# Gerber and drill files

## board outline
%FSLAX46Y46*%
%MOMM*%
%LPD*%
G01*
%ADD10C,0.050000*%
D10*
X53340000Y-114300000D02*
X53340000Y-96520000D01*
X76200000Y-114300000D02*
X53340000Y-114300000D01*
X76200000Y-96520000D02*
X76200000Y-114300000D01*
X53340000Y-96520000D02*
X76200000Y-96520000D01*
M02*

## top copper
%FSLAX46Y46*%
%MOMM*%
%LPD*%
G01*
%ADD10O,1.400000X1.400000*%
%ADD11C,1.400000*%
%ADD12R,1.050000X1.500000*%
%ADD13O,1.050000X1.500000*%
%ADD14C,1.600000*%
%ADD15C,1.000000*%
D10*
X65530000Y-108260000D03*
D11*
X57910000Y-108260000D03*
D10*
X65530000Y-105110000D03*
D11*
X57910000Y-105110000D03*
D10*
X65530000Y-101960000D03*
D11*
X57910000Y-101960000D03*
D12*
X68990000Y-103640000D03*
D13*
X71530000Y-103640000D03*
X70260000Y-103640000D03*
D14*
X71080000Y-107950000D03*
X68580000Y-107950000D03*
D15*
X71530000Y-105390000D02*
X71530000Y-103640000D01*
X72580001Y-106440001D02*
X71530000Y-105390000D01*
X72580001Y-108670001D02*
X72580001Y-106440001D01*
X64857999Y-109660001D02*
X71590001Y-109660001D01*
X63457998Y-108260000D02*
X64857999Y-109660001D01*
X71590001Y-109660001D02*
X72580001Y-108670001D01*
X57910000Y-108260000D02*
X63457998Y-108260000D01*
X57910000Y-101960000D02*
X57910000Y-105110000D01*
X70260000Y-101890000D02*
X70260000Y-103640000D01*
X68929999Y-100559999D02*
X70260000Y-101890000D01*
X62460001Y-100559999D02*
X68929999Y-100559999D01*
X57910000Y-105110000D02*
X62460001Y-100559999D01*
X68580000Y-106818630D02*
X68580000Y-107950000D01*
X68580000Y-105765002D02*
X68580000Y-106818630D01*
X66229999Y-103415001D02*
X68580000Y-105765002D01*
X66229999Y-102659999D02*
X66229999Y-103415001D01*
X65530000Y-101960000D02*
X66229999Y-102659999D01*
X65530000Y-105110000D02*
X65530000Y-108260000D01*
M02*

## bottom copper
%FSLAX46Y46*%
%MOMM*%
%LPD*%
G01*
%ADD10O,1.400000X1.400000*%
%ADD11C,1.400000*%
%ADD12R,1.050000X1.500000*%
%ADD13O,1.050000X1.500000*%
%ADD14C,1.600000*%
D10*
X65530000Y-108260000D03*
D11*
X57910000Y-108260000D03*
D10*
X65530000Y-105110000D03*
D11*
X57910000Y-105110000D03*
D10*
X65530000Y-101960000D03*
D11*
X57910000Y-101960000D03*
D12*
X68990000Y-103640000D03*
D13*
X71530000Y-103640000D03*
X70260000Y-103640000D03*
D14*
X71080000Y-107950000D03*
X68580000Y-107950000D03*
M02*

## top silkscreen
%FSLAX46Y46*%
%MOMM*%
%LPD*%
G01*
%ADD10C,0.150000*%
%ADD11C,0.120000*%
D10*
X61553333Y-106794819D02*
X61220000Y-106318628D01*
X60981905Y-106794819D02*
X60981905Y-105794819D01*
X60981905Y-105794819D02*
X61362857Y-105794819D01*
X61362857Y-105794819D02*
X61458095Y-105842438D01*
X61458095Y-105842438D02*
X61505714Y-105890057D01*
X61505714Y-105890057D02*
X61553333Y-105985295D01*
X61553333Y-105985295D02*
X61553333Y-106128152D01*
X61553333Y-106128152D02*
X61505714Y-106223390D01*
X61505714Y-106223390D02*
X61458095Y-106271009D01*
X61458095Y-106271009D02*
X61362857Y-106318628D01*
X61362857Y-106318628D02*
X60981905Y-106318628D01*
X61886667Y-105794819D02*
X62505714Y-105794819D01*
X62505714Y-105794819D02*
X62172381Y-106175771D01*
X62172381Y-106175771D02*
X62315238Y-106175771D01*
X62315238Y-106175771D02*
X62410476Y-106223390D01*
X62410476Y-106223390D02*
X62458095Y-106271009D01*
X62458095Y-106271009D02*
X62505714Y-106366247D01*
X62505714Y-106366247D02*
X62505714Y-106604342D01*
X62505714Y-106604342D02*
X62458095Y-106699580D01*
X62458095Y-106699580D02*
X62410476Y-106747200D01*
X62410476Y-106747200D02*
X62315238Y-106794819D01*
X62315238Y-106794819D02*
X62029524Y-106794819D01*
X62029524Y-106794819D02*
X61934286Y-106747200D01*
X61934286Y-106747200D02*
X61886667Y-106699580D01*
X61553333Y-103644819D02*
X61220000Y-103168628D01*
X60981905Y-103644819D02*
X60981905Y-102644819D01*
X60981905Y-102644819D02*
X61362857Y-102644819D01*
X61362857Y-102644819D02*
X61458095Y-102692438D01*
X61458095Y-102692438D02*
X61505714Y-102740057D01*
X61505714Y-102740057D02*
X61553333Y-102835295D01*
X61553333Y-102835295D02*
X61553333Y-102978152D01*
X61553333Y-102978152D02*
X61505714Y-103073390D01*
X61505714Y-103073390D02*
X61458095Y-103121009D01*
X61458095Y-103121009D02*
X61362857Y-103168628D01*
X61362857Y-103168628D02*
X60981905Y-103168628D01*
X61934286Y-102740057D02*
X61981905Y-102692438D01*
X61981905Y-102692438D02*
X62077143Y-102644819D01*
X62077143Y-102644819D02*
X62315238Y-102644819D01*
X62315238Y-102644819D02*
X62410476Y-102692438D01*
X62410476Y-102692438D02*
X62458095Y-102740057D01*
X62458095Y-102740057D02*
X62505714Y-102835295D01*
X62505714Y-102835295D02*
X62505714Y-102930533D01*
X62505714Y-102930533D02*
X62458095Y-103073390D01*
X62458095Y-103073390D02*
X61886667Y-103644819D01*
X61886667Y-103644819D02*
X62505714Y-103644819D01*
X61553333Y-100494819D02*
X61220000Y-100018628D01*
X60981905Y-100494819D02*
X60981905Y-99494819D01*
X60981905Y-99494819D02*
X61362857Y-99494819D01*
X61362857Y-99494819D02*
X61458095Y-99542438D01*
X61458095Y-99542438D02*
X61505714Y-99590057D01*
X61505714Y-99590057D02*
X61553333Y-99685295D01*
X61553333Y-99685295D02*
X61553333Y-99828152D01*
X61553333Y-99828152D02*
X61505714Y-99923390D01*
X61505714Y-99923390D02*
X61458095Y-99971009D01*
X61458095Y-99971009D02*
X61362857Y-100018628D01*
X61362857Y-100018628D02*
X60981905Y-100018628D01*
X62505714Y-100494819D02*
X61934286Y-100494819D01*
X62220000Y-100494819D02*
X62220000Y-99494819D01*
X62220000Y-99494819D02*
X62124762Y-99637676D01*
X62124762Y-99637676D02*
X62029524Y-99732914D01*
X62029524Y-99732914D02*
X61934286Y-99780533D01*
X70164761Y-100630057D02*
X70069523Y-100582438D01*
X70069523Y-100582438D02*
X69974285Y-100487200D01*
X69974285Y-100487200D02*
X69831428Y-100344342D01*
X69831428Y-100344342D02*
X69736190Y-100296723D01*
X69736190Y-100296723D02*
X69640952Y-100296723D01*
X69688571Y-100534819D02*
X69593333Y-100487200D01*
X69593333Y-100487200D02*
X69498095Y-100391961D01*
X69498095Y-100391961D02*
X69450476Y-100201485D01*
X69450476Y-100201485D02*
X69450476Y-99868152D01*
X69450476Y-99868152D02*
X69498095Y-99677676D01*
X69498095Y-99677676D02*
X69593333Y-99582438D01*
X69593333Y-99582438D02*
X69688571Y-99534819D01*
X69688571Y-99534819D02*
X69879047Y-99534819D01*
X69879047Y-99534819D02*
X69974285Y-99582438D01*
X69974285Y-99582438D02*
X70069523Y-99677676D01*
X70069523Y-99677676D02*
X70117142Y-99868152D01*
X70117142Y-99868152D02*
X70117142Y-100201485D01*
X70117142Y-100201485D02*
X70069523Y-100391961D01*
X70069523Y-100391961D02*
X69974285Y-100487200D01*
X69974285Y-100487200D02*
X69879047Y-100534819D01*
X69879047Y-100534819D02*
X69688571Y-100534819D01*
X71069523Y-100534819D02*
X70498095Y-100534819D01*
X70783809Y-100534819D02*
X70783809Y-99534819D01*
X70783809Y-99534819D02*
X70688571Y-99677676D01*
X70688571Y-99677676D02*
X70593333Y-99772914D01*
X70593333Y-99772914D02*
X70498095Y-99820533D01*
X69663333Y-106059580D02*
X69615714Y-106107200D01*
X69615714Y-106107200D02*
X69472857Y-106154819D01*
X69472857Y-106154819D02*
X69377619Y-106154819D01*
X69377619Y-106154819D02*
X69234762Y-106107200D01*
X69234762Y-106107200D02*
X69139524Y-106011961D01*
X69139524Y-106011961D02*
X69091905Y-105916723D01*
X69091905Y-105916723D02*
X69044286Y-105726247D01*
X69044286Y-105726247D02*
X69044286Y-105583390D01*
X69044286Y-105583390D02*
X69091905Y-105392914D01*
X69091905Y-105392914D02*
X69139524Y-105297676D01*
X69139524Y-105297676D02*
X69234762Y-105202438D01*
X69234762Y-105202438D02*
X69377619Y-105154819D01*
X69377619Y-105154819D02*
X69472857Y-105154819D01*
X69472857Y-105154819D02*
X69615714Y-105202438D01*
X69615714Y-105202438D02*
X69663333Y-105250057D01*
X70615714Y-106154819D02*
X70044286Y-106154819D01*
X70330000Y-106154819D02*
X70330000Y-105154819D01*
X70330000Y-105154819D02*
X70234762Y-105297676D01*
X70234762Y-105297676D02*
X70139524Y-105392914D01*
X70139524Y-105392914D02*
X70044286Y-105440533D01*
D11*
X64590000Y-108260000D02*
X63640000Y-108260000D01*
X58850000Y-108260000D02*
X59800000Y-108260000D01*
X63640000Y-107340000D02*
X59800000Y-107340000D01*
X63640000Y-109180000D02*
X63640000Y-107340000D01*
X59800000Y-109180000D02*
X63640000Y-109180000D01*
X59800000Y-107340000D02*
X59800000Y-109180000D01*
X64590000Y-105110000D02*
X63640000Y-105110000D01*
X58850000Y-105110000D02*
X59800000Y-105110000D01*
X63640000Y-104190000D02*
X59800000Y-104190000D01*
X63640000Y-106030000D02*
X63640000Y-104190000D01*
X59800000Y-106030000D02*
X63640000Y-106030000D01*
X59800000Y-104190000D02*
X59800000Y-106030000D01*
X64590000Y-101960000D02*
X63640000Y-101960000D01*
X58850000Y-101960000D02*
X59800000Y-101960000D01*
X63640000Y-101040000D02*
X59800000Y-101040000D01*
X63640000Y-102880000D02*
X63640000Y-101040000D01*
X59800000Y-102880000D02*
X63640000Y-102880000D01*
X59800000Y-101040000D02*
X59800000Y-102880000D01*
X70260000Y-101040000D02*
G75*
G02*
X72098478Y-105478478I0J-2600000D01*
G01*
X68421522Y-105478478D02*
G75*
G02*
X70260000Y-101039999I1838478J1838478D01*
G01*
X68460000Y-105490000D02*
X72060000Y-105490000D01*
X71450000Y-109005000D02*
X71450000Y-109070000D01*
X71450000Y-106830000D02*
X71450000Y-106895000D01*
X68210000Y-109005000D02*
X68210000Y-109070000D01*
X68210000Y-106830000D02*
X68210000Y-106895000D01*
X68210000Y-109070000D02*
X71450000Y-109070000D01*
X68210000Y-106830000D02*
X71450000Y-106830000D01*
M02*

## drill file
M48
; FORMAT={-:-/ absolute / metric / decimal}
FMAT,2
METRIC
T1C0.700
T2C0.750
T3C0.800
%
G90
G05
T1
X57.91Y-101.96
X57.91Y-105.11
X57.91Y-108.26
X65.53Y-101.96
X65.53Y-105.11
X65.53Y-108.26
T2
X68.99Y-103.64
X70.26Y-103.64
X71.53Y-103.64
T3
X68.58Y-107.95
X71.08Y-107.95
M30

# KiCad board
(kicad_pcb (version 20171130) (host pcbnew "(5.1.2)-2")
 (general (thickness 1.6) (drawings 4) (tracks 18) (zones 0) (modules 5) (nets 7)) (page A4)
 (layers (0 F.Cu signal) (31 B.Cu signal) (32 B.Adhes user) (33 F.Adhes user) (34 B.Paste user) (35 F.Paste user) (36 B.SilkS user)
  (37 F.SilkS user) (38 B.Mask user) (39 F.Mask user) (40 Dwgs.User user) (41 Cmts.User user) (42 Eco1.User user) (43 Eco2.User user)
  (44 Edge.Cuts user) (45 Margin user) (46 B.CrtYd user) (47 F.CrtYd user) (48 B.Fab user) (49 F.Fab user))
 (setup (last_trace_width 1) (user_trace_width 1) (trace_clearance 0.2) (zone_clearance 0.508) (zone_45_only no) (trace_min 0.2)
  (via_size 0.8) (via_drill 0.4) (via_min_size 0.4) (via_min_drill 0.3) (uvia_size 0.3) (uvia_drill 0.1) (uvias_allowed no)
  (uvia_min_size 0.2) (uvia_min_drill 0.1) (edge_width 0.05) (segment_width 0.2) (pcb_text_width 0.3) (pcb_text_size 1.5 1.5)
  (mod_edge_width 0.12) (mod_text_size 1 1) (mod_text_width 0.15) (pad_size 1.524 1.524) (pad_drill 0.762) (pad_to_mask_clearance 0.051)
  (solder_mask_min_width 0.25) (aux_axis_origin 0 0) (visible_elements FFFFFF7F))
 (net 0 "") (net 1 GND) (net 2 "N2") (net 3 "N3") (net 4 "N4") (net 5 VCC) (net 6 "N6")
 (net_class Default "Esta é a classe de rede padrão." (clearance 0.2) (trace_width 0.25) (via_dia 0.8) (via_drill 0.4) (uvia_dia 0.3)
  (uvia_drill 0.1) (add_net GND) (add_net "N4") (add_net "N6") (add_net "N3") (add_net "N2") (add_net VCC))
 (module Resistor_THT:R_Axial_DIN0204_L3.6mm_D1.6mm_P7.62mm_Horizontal (layer F.Cu) (at 57.91 108.26)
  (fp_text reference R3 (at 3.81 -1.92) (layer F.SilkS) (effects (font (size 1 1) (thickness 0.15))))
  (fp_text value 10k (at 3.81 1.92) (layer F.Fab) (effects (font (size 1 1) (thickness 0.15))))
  (fp_line (start 6.68 0) (end 5.73 0) (layer F.SilkS) (width 0.12))
  (fp_line (start 0.94 0) (end 1.89 0) (layer F.SilkS) (width 0.12))
  (fp_line (start 5.73 -0.92) (end 1.89 -0.92) (layer F.SilkS) (width 0.12))
  (fp_line (start 5.73 0.92) (end 5.73 -0.92) (layer F.SilkS) (width 0.12))
  (fp_line (start 1.89 0.92) (end 5.73 0.92) (layer F.SilkS) (width 0.12))
  (fp_line (start 1.89 -0.92) (end 1.89 0.92) (layer F.SilkS) (width 0.12))
  (pad 2 thru_hole oval (at 7.62 0) (size 1.4 1.4) (drill 0.7) (layers *.Cu *.Mask) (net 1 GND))
  (pad 1 thru_hole circle (at 0 0) (size 1.4 1.4) (drill 0.7) (layers *.Cu *.Mask) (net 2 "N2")))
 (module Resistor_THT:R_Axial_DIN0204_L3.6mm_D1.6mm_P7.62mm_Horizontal (layer F.Cu) (at 57.91 105.11)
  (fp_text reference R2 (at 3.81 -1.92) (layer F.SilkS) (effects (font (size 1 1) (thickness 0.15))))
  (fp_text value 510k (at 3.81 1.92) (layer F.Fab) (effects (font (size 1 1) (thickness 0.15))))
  (fp_line (start 6.68 0) (end 5.73 0) (layer F.SilkS) (width 0.12))
  (fp_line (start 0.94 0) (end 1.89 0) (layer F.SilkS) (width 0.12))
  (fp_line (start 5.73 -0.92) (end 1.89 -0.92) (layer F.SilkS) (width 0.12))
  (fp_line (start 5.73 0.92) (end 5.73 -0.92) (layer F.SilkS) (width 0.12))
  (fp_line (start 1.89 0.92) (end 5.73 0.92) (layer F.SilkS) (width 0.12))
  (fp_line (start 1.89 -0.92) (end 1.89 0.92) (layer F.SilkS) (width 0.12))
  (pad 2 thru_hole oval (at 7.62 0) (size 1.4 1.4) (drill 0.7) (layers *.Cu *.Mask) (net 1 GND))
  (pad 1 thru_hole circle (at 0 0) (size 1.4 1.4) (drill 0.7) (layers *.Cu *.Mask) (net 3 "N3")))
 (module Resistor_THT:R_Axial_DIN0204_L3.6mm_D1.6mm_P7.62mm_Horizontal (layer F.Cu) (at 57.91 101.96)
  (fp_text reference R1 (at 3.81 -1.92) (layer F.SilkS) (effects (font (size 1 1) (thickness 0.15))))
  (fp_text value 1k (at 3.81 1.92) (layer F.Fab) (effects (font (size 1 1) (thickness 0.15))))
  (fp_line (start 6.68 0) (end 5.73 0) (layer F.SilkS) (width 0.12))
  (fp_line (start 0.94 0) (end 1.89 0) (layer F.SilkS) (width 0.12))
  (fp_line (start 5.73 -0.92) (end 1.89 -0.92) (layer F.SilkS) (width 0.12))
  (fp_line (start 5.73 0.92) (end 5.73 -0.92) (layer F.SilkS) (width 0.12))
  (fp_line (start 1.89 0.92) (end 5.73 0.92) (layer F.SilkS) (width 0.12))
  (fp_line (start 1.89 -0.92) (end 1.89 0.92) (layer F.SilkS) (width 0.12))
  (pad 2 thru_hole oval (at 7.62 0) (size 1.4 1.4) (drill 0.7) (layers *.Cu *.Mask) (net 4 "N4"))
  (pad 1 thru_hole circle (at 0 0) (size 1.4 1.4) (drill 0.7) (layers *.Cu *.Mask) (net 3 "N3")))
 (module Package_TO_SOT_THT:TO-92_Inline (layer F.Cu) (at 68.99 103.64)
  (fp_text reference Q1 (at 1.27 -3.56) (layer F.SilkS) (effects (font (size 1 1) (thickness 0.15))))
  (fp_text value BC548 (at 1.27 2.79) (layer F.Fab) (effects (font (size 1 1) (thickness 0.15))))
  (fp_arc (start 1.27 0) (end 1.27 -2.6) (angle 135) (layer F.SilkS) (width 0.12))
  (fp_arc (start 1.27 0) (end 1.27 -2.6) (angle -135) (layer F.SilkS) (width 0.12))
  (fp_line (start -0.53 1.85) (end 3.07 1.85) (layer F.SilkS) (width 0.12))
  (pad 1 thru_hole rect (at 0 0) (size 1.05 1.5) (drill 0.75) (layers *.Cu *.Mask) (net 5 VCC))
  (pad 3 thru_hole oval (at 2.54 0) (size 1.05 1.5) (drill 0.75) (layers *.Cu *.Mask) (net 2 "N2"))
  (pad 2 thru_hole oval (at 1.27 0) (size 1.05 1.5) (drill 0.75) (layers *.Cu *.Mask) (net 3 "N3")))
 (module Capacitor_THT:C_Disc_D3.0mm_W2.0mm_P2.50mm (layer F.Cu) (at 68.58 107.95)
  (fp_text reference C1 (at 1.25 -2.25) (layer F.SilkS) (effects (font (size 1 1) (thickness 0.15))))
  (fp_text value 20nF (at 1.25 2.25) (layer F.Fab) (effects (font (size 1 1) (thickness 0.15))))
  (fp_line (start 2.87 1.055) (end 2.87 1.12) (layer F.SilkS) (width 0.12))
  (fp_line (start 2.87 -1.12) (end 2.87 -1.055) (layer F.SilkS) (width 0.12))
  (fp_line (start -0.37 1.055) (end -0.37 1.12) (layer F.SilkS) (width 0.12))
  (fp_line (start -0.37 -1.12) (end -0.37 -1.055) (layer F.SilkS) (width 0.12))
  (fp_line (start -0.37 1.12) (end 2.87 1.12) (layer F.SilkS) (width 0.12))
  (fp_line (start -0.37 -1.12) (end 2.87 -1.12) (layer F.SilkS) (width 0.12))
  (pad 2 thru_hole circle (at 2.5 0) (size 1.6 1.6) (drill 0.8) (layers *.Cu *.Mask) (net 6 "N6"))
  (pad 1 thru_hole circle (at 0 0) (size 1.6 1.6) (drill 0.8) (layers *.Cu *.Mask) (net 4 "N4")))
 (gr_line (start 53.34 114.3) (end 53.34 96.52) (layer Edge.Cuts) (width 0.05))
 (gr_line (start 76.2 114.3) (end 53.34 114.3) (layer Edge.Cuts) (width 0.05))
 (gr_line (start 76.2 96.52) (end 76.2 114.3) (layer Edge.Cuts) (width 0.05))
 (gr_line (start 53.34 96.52) (end 76.2 96.52) (layer Edge.Cuts) (width 0.05))
 (segment (start 71.53 105.39) (end 71.53 103.64) (width 1) (layer F.Cu) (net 2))
 (segment (start 72.580001 106.440001) (end 71.53 105.39) (width 1) (layer F.Cu) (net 2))
 (segment (start 72.580001 108.670001) (end 72.580001 106.440001) (width 1) (layer F.Cu) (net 2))
 (segment (start 64.857999 109.660001) (end 71.590001 109.660001) (width 1) (layer F.Cu) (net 2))
 (segment (start 63.457998 108.26) (end 64.857999 109.660001) (width 1) (layer F.Cu) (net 2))
 (segment (start 71.590001 109.660001) (end 72.580001 108.670001) (width 1) (layer F.Cu) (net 2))
 (segment (start 57.91 108.26) (end 63.457998 108.26) (width 1) (layer F.Cu) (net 2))
 (segment (start 57.91 101.96) (end 57.91 105.11) (width 1) (layer F.Cu) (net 3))
 (segment (start 70.26 101.89) (end 70.26 103.64) (width 1) (layer F.Cu) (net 3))
 (segment (start 68.929999 100.559999) (end 70.26 101.89) (width 1) (layer F.Cu) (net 3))
 (segment (start 62.460001 100.559999) (end 68.929999 100.559999) (width 1) (layer F.Cu) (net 3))
 (segment (start 57.91 105.11) (end 62.460001 100.559999) (width 1) (layer F.Cu) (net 3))
 (segment (start 68.58 106.81863) (end 68.58 107.95) (width 1) (layer F.Cu) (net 4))
 (segment (start 68.58 105.765002) (end 68.58 106.81863) (width 1) (layer F.Cu) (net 4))
 (segment (start 66.229999 103.415001) (end 68.58 105.765002) (width 1) (layer F.Cu) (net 4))
 (segment (start 66.229999 102.659999) (end 66.229999 103.415001) (width 1) (layer F.Cu) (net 4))
 (segment (start 65.53 101.96) (end 66.229999 102.659999) (width 1) (layer F.Cu) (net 4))
 (segment (start 65.53 105.11) (end 65.53 108.26) (width 1) (layer F.Cu) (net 1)))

